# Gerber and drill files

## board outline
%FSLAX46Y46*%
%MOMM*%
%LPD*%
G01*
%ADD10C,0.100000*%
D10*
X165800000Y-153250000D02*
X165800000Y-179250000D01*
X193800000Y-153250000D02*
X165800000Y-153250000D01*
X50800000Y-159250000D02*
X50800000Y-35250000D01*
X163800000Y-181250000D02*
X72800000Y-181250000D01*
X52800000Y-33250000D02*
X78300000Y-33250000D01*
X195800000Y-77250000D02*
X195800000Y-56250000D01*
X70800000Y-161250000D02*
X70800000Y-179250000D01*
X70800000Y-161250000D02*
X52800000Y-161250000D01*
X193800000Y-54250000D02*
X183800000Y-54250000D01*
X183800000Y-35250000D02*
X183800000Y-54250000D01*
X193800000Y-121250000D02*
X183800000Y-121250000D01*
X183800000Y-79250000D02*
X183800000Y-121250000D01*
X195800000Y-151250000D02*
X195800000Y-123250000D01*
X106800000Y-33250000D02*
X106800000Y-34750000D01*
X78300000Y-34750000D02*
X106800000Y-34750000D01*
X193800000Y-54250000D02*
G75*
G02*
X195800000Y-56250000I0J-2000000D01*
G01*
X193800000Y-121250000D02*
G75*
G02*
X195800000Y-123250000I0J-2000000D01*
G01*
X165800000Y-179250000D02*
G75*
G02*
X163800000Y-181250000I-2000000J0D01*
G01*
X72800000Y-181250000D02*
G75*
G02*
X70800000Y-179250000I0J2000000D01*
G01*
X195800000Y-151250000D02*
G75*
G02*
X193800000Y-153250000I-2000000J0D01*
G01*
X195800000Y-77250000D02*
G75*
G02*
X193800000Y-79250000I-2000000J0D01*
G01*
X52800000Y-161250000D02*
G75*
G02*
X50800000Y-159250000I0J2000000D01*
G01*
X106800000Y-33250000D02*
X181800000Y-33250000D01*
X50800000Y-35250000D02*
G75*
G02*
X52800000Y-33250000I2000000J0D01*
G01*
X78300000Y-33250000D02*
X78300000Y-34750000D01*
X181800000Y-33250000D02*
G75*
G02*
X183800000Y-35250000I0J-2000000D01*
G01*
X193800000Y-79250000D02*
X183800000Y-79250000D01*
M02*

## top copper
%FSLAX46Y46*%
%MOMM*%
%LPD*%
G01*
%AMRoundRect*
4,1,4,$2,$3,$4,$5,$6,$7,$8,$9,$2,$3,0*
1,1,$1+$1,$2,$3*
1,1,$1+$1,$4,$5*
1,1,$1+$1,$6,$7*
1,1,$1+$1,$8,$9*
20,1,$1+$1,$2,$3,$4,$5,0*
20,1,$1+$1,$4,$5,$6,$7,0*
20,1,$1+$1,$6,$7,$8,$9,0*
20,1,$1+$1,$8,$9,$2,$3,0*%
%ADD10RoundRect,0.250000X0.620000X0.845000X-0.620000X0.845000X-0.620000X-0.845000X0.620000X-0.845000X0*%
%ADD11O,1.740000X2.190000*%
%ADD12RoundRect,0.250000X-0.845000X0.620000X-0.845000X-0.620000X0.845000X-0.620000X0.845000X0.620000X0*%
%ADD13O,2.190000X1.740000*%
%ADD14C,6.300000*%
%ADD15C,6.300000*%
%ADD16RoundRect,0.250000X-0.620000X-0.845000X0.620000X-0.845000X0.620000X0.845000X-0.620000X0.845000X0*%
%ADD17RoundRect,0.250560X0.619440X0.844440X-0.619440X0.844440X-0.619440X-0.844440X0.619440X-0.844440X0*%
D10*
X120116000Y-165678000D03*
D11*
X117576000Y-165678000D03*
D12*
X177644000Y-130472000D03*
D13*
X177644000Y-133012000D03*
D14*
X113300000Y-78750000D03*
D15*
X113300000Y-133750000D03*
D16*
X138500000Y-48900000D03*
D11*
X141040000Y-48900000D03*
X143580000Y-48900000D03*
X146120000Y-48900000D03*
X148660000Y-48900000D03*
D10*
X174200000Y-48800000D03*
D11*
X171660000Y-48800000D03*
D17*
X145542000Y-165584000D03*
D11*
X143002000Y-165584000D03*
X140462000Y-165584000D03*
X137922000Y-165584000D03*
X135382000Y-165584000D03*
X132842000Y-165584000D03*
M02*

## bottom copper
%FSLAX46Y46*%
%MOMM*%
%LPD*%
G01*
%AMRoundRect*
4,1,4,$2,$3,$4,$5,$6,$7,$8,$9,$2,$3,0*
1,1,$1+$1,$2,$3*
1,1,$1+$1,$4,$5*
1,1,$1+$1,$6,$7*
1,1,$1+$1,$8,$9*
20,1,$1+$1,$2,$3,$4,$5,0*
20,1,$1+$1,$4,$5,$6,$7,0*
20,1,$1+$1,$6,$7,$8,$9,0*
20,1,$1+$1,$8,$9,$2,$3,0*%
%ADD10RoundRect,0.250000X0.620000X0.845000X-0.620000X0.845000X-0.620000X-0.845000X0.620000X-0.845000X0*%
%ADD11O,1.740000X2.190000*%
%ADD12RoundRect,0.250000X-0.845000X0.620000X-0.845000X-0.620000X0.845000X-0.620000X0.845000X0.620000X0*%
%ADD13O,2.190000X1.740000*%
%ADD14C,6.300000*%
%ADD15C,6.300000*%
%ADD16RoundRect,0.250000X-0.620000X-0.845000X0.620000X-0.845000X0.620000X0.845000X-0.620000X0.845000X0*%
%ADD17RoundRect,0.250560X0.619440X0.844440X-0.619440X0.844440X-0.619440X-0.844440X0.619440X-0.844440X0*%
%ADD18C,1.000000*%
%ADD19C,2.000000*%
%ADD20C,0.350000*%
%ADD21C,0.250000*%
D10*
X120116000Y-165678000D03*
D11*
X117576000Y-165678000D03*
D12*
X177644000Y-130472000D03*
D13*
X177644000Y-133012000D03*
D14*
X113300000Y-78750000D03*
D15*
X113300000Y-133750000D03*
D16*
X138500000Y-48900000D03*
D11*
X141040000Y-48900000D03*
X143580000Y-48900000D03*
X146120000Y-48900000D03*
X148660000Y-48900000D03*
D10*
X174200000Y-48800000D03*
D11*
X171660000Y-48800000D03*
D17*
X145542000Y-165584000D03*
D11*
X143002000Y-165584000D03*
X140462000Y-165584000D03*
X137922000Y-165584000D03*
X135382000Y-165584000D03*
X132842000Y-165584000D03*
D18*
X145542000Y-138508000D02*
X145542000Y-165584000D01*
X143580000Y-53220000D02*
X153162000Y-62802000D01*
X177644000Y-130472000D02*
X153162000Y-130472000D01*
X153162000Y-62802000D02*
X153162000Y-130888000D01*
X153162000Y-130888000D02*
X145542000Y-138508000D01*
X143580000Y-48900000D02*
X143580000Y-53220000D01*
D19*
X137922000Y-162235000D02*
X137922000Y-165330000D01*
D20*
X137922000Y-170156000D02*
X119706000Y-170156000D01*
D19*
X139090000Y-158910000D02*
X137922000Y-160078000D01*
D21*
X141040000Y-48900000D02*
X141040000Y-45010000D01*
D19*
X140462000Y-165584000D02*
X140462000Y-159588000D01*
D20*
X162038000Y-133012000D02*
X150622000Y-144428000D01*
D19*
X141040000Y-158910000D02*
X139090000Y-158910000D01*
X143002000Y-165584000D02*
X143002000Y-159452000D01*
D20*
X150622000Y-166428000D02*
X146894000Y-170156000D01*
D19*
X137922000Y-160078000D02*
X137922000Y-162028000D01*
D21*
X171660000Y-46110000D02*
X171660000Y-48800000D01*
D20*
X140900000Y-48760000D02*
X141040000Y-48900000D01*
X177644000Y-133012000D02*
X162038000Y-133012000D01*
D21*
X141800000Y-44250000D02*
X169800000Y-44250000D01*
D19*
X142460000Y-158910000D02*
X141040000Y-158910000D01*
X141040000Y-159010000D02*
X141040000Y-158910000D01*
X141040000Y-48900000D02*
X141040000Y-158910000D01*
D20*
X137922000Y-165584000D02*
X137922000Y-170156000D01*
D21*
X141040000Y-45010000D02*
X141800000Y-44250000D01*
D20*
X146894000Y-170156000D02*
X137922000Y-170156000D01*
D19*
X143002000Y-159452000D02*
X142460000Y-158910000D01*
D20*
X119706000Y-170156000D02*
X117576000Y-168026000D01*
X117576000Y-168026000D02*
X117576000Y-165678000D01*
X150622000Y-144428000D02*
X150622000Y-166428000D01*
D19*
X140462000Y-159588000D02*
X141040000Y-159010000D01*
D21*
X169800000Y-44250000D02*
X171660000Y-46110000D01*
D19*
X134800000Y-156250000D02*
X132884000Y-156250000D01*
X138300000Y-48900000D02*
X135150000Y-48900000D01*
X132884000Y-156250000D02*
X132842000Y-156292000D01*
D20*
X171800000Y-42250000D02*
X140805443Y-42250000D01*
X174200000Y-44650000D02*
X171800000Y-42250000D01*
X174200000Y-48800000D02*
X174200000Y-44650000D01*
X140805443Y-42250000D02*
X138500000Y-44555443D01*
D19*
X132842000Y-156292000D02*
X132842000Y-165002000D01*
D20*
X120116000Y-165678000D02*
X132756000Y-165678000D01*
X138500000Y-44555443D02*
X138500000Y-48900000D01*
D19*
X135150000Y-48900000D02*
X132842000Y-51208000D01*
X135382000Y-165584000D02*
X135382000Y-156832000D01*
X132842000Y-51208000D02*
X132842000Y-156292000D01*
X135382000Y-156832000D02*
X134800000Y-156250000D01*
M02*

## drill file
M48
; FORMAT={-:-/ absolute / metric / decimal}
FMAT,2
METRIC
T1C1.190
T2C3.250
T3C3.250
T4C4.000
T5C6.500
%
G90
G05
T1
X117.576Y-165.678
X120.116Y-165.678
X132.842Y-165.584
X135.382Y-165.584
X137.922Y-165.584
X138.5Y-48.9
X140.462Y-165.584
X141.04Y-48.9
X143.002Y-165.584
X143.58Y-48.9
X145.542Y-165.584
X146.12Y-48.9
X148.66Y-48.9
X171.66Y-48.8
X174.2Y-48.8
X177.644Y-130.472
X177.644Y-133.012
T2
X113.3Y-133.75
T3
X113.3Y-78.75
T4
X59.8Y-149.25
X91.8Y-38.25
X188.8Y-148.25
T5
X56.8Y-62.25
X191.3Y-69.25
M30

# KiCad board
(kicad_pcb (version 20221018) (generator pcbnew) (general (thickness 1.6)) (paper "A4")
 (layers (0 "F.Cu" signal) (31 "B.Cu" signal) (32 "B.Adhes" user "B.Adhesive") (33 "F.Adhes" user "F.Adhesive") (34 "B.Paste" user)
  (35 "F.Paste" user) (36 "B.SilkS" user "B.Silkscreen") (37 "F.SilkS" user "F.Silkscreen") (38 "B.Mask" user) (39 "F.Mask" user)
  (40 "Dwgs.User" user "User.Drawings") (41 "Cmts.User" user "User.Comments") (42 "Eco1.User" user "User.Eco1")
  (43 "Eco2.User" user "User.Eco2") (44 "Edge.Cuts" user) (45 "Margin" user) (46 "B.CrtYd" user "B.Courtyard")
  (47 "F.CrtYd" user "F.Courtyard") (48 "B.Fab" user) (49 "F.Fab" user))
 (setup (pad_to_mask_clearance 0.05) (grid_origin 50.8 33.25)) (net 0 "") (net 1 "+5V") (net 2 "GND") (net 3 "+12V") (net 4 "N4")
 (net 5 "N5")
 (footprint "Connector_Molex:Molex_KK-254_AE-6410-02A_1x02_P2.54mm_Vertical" (layer "F.Cu") (at 120.116 165.678 180)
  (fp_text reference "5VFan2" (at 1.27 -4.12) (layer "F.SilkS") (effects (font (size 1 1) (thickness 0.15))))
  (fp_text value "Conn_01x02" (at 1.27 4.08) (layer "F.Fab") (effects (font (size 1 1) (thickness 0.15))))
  (pad "1" thru_hole roundrect (at 0 0 180) (size 1.74 2.19) (drill 1.19) (layers "*.Cu" "*.Mask") (roundrect_rratio 0.143678) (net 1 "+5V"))
  (pad "2" thru_hole oval (at 2.54 0 180) (size 1.74 2.19) (drill 1.19) (layers "*.Cu" "*.Mask") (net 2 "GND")))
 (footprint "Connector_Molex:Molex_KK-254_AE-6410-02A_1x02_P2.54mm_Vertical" (layer "F.Cu") (at 177.644 130.472 -90)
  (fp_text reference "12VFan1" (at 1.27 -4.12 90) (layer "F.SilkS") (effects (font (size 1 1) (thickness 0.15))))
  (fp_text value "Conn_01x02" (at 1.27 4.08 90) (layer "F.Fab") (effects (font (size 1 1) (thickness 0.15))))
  (pad "1" thru_hole roundrect (at 0 0 270) (size 1.74 2.19) (drill 1.19) (layers "*.Cu" "*.Mask") (roundrect_rratio 0.143678)
   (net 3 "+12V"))
  (pad "2" thru_hole oval (at 2.54 0 270) (size 1.74 2.19) (drill 1.19) (layers "*.Cu" "*.Mask") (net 2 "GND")))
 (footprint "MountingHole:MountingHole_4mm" (layer "F.Cu") (at 188.8 148.25 180)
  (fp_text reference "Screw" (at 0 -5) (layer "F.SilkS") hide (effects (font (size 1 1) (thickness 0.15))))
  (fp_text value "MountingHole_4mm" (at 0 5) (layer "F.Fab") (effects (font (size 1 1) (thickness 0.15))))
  (pad "" np_thru_hole circle (at 0 0 180) (size 4 4) (drill 4) (layers "*.Cu" "*.Mask")))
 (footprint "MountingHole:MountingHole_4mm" (layer "F.Cu") (at 91.8 38.25 180)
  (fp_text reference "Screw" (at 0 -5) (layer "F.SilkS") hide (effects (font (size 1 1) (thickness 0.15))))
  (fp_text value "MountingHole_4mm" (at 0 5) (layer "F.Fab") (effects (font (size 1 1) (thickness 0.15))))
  (pad "" np_thru_hole circle (at 0 0 180) (size 4 4) (drill 4) (layers "*.Cu" "*.Mask")))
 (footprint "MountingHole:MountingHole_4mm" (layer "F.Cu") (at 59.8 149.25 180)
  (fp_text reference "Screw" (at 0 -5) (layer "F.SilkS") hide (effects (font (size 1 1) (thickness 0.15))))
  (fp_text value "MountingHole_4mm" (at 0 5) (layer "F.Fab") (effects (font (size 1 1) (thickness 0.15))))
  (pad "" np_thru_hole circle (at 0 0 180) (size 4 4) (drill 4) (layers "*.Cu" "*.Mask")))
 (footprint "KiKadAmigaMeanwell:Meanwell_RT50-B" (layer "F.Cu") (at 122.8 107.25 -90)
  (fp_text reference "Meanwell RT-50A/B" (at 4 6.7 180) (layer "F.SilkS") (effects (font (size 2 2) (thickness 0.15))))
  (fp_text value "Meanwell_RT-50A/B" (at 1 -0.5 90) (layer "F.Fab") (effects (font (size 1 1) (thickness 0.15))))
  (pad "" np_thru_hole circle (at -28.5 9.5 270) (size 6.3 6.3) (drill 3.25) (layers "*.Cu" "*.Mask"))
  (pad "" thru_hole circle (at 26.5 9.5 270) (size 6.3 6.3) (drill 3.25) (layers "*.Cu" "*.Mask")))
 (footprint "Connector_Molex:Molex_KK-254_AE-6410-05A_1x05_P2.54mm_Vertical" (layer "F.Cu") (at 138.5 48.9)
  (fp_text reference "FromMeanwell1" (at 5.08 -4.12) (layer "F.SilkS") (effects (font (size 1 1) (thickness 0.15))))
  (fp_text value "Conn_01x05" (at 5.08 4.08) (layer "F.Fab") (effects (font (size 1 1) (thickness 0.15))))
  (pad "1" thru_hole roundrect (at 0 0) (size 1.74 2.19) (drill 1.19) (layers "*.Cu" "*.Mask") (roundrect_rratio 0.143678) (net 1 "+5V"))
  (pad "2" thru_hole oval (at 2.54 0) (size 1.74 2.19) (drill 1.19) (layers "*.Cu" "*.Mask") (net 2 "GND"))
  (pad "3" thru_hole oval (at 5.08 0) (size 1.74 2.19) (drill 1.19) (layers "*.Cu" "*.Mask") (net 3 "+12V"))
  (pad "4" thru_hole oval (at 7.62 0) (size 1.74 2.19) (drill 1.19) (layers "*.Cu" "*.Mask") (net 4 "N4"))
  (pad "5" thru_hole oval (at 10.16 0) (size 1.74 2.19) (drill 1.19) (layers "*.Cu" "*.Mask") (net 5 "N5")))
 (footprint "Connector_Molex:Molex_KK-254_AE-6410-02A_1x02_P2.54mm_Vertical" (layer "F.Cu") (at 174.2 48.8 180)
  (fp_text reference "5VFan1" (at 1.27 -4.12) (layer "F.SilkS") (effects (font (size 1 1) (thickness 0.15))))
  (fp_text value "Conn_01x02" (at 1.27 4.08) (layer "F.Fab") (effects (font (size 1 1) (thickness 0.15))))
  (pad "1" thru_hole roundrect (at 0 0 180) (size 1.74 2.19) (drill 1.19) (layers "*.Cu" "*.Mask") (roundrect_rratio 0.143678) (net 1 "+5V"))
  (pad "2" thru_hole oval (at 2.54 0 180) (size 1.74 2.19) (drill 1.19) (layers "*.Cu" "*.Mask") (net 2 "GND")))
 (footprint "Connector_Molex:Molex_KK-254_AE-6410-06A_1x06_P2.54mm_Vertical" (layer "F.Cu") (at 145.542 165.584 180)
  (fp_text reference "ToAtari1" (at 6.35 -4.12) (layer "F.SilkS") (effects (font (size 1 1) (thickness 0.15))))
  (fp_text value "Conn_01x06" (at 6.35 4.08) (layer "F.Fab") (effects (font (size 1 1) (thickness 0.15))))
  (pad "1" thru_hole roundrect (at 0 0 180) (size 1.74 2.19) (drill 1.19) (layers "*.Cu" "*.Mask") (roundrect_rratio 0.144) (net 3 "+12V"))
  (pad "2" thru_hole oval (at 2.54 0 180) (size 1.74 2.19) (drill 1.19) (layers "*.Cu" "*.Mask") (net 2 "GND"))
  (pad "3" thru_hole oval (at 5.08 0 180) (size 1.74 2.19) (drill 1.19) (layers "*.Cu" "*.Mask") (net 2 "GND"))
  (pad "4" thru_hole oval (at 7.62 0 180) (size 1.74 2.19) (drill 1.19) (layers "*.Cu" "*.Mask") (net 2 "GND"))
  (pad "5" thru_hole oval (at 10.16 0 180) (size 1.74 2.19) (drill 1.19) (layers "*.Cu" "*.Mask") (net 1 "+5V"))
  (pad "6" thru_hole oval (at 12.7 0 180) (size 1.74 2.19) (drill 1.19) (layers "*.Cu" "*.Mask") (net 1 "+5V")))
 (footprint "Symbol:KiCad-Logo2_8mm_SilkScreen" (layer "F.Cu") (at 64.77 41.124)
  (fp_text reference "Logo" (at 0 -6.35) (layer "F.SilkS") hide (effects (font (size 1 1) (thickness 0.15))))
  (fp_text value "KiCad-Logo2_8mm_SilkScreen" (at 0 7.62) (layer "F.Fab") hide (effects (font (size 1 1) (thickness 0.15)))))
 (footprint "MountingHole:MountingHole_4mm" (layer "F.Cu") (at 56.8 62.25 180)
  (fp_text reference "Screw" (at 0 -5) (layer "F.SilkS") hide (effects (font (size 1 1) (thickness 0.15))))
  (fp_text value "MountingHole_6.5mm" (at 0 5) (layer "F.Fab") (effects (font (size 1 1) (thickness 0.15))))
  (pad "" np_thru_hole circle (at 0 0 180) (size 6.5 6.5) (drill 6.5) (layers "*.Cu" "*.Mask")))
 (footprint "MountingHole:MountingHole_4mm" (layer "F.Cu") (at 191.3 69.25 180)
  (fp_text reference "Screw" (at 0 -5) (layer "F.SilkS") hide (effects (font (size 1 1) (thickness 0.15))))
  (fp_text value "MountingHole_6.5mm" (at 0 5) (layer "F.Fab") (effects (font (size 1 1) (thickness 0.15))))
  (pad "" np_thru_hole circle (at 0 0 180) (size 6.5 6.5) (drill 6.5) (layers "*.Cu" "*.Mask")))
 (gr_line (start 165.8 153.25) (end 165.8 179.25) (stroke (width 0.1) (type solid)) (layer "Edge.Cuts"))
 (gr_line (start 193.8 153.25) (end 165.8 153.25) (stroke (width 0.1) (type solid)) (layer "Edge.Cuts"))
 (gr_line (start 50.8 159.25) (end 50.8 35.25) (stroke (width 0.1) (type solid)) (layer "Edge.Cuts"))
 (gr_line (start 163.8 181.25) (end 72.8 181.25) (stroke (width 0.1) (type solid)) (layer "Edge.Cuts"))
 (gr_line (start 52.8 33.25) (end 78.3 33.25) (stroke (width 0.1) (type solid)) (layer "Edge.Cuts"))
 (gr_line (start 195.8 77.25) (end 195.8 56.25) (stroke (width 0.1) (type solid)) (layer "Edge.Cuts"))
 (gr_line (start 70.8 161.25) (end 70.8 179.25) (stroke (width 0.1) (type solid)) (layer "Edge.Cuts"))
 (gr_line (start 70.8 161.25) (end 52.8 161.25) (stroke (width 0.1) (type solid)) (layer "Edge.Cuts"))
 (gr_line (start 193.8 54.25) (end 183.8 54.25) (stroke (width 0.1) (type solid)) (layer "Edge.Cuts"))
 (gr_line (start 183.8 35.25) (end 183.8 54.25) (stroke (width 0.1) (type solid)) (layer "Edge.Cuts"))
 (gr_line (start 193.8 121.25) (end 183.8 121.25) (stroke (width 0.1) (type solid)) (layer "Edge.Cuts"))
 (gr_line (start 183.8 79.25) (end 183.8 121.25) (stroke (width 0.1) (type solid)) (layer "Edge.Cuts"))
 (gr_line (start 195.8 151.25) (end 195.8 123.25) (stroke (width 0.1) (type solid)) (layer "Edge.Cuts"))
 (gr_line (start 106.8 33.25) (end 106.8 34.75) (stroke (width 0.1) (type solid)) (layer "Edge.Cuts"))
 (gr_line (start 78.3 34.75) (end 106.8 34.75) (stroke (width 0.1) (type solid)) (layer "Edge.Cuts"))
 (gr_arc (start 193.8 54.25) (mid 195.214214 54.835786) (end 195.8 56.25) (stroke (width 0.1) (type solid)) (layer "Edge.Cuts"))
 (gr_arc (start 193.8 121.25) (mid 195.214214 121.835786) (end 195.8 123.25) (stroke (width 0.1) (type solid)) (layer "Edge.Cuts"))
 (gr_arc (start 165.8 179.25) (mid 165.214214 180.664214) (end 163.8 181.25) (stroke (width 0.1) (type solid)) (layer "Edge.Cuts"))
 (gr_arc (start 72.8 181.25) (mid 71.385786 180.664214) (end 70.8 179.25) (stroke (width 0.1) (type solid)) (layer "Edge.Cuts"))
 (gr_arc (start 195.8 151.25) (mid 195.214214 152.664214) (end 193.8 153.25) (stroke (width 0.1) (type solid)) (layer "Edge.Cuts"))
 (gr_arc (start 195.8 77.25) (mid 195.214214 78.664214) (end 193.8 79.25) (stroke (width 0.1) (type solid)) (layer "Edge.Cuts"))
 (gr_arc (start 52.8 161.25) (mid 51.385786 160.664214) (end 50.8 159.25) (stroke (width 0.1) (type solid)) (layer "Edge.Cuts"))
 (gr_line (start 106.8 33.25) (end 181.8 33.25) (stroke (width 0.1) (type solid)) (layer "Edge.Cuts"))
 (gr_arc (start 50.8 35.25) (mid 51.385786 33.835786) (end 52.8 33.25) (stroke (width 0.1) (type solid)) (layer "Edge.Cuts"))
 (gr_line (start 78.3 33.25) (end 78.3 34.75) (stroke (width 0.1) (type solid)) (layer "Edge.Cuts"))
 (gr_arc (start 181.8 33.25) (mid 183.214214 33.835786) (end 183.8 35.25) (stroke (width 0.1) (type solid)) (layer "Edge.Cuts"))
 (gr_line (start 193.8 79.25) (end 183.8 79.25) (stroke (width 0.1) (type solid)) (layer "Edge.Cuts"))
 (segment (start 145.542 138.508) (end 145.542 165.584) (width 1) (layer "B.Cu") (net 3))
 (segment (start 143.58 53.22) (end 153.162 62.802) (width 1) (layer "B.Cu") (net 3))
 (segment (start 177.644 130.472) (end 153.162 130.472) (width 1) (layer "B.Cu") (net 3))
 (segment (start 153.162 62.802) (end 153.162 130.888) (width 1) (layer "B.Cu") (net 3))
 (segment (start 153.162 130.888) (end 145.542 138.508) (width 1) (layer "B.Cu") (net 3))
 (segment (start 143.58 48.9) (end 143.58 53.22) (width 1) (layer "B.Cu") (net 3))
 (segment (start 137.922 162.235) (end 137.922 165.33) (width 2) (layer "B.Cu") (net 2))
 (segment (start 137.922 170.156) (end 119.706 170.156) (width 0.35) (layer "B.Cu") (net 2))
 (segment (start 139.09 158.91) (end 137.922 160.078) (width 2) (layer "B.Cu") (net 2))
 (segment (start 141.04 48.9) (end 141.04 45.01) (width 0.25) (layer "B.Cu") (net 2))
 (segment (start 140.462 165.584) (end 140.462 159.588) (width 2) (layer "B.Cu") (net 2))
 (segment (start 162.038 133.012) (end 150.622 144.428) (width 0.35) (layer "B.Cu") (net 2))
 (segment (start 141.04 158.91) (end 139.09 158.91) (width 2) (layer "B.Cu") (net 2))
 (segment (start 143.002 165.584) (end 143.002 159.452) (width 2) (layer "B.Cu") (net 2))
 (segment (start 150.622 166.428) (end 146.894 170.156) (width 0.35) (layer "B.Cu") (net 2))
 (segment (start 137.922 160.078) (end 137.922 162.028) (width 2) (layer "B.Cu") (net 2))
 (segment (start 171.66 46.11) (end 171.66 48.8) (width 0.25) (layer "B.Cu") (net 2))
 (segment (start 140.9 48.76) (end 141.04 48.9) (width 0.35) (layer "B.Cu") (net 2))
 (segment (start 177.644 133.012) (end 162.038 133.012) (width 0.35) (layer "B.Cu") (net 2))
 (segment (start 141.8 44.25) (end 169.8 44.25) (width 0.25) (layer "B.Cu") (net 2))
 (segment (start 142.46 158.91) (end 141.04 158.91) (width 2) (layer "B.Cu") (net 2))
 (segment (start 141.04 159.01) (end 141.04 158.91) (width 2) (layer "B.Cu") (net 2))
 (segment (start 141.04 48.9) (end 141.04 158.91) (width 2) (layer "B.Cu") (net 2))
 (segment (start 137.922 165.584) (end 137.922 170.156) (width 0.35) (layer "B.Cu") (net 2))
 (segment (start 141.04 45.01) (end 141.8 44.25) (width 0.25) (layer "B.Cu") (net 2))
 (segment (start 146.894 170.156) (end 137.922 170.156) (width 0.35) (layer "B.Cu") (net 2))
 (segment (start 143.002 159.452) (end 142.46 158.91) (width 2) (layer "B.Cu") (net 2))
 (segment (start 119.706 170.156) (end 117.576 168.026) (width 0.35) (layer "B.Cu") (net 2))
 (segment (start 117.576 168.026) (end 117.576 165.678) (width 0.35) (layer "B.Cu") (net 2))
 (segment (start 150.622 144.428) (end 150.622 166.428) (width 0.35) (layer "B.Cu") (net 2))
 (segment (start 140.462 159.588) (end 141.04 159.01) (width 2) (layer "B.Cu") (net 2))
 (segment (start 169.8 44.25) (end 171.66 46.11) (width 0.25) (layer "B.Cu") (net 2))
 (segment (start 134.8 156.25) (end 132.884 156.25) (width 2) (layer "B.Cu") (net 1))
 (segment (start 138.3 48.9) (end 135.15 48.9) (width 2) (layer "B.Cu") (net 1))
 (segment (start 132.884 156.25) (end 132.842 156.292) (width 2) (layer "B.Cu") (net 1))
 (segment (start 171.8 42.25) (end 140.805443 42.25) (width 0.35) (layer "B.Cu") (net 1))
 (segment (start 174.2 44.65) (end 171.8 42.25) (width 0.35) (layer "B.Cu") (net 1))
 (segment (start 174.2 48.8) (end 174.2 44.65) (width 0.35) (layer "B.Cu") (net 1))
 (segment (start 140.805443 42.25) (end 138.5 44.555443) (width 0.35) (layer "B.Cu") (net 1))
 (segment (start 132.842 156.292) (end 132.842 165.002) (width 2) (layer "B.Cu") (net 1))
 (segment (start 120.116 165.678) (end 132.756 165.678) (width 0.35) (layer "B.Cu") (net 1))
 (segment (start 138.5 44.555443) (end 138.5 48.9) (width 0.35) (layer "B.Cu") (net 1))
 (segment (start 135.15 48.9) (end 132.842 51.208) (width 2) (layer "B.Cu") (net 1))
 (segment (start 135.382 165.584) (end 135.382 156.832) (width 2) (layer "B.Cu") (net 1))
 (segment (start 132.842 51.208) (end 132.842 156.292) (width 2) (layer "B.Cu") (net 1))
 (segment (start 135.382 156.832) (end 134.8 156.25) (width 2) (layer "B.Cu") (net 1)))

